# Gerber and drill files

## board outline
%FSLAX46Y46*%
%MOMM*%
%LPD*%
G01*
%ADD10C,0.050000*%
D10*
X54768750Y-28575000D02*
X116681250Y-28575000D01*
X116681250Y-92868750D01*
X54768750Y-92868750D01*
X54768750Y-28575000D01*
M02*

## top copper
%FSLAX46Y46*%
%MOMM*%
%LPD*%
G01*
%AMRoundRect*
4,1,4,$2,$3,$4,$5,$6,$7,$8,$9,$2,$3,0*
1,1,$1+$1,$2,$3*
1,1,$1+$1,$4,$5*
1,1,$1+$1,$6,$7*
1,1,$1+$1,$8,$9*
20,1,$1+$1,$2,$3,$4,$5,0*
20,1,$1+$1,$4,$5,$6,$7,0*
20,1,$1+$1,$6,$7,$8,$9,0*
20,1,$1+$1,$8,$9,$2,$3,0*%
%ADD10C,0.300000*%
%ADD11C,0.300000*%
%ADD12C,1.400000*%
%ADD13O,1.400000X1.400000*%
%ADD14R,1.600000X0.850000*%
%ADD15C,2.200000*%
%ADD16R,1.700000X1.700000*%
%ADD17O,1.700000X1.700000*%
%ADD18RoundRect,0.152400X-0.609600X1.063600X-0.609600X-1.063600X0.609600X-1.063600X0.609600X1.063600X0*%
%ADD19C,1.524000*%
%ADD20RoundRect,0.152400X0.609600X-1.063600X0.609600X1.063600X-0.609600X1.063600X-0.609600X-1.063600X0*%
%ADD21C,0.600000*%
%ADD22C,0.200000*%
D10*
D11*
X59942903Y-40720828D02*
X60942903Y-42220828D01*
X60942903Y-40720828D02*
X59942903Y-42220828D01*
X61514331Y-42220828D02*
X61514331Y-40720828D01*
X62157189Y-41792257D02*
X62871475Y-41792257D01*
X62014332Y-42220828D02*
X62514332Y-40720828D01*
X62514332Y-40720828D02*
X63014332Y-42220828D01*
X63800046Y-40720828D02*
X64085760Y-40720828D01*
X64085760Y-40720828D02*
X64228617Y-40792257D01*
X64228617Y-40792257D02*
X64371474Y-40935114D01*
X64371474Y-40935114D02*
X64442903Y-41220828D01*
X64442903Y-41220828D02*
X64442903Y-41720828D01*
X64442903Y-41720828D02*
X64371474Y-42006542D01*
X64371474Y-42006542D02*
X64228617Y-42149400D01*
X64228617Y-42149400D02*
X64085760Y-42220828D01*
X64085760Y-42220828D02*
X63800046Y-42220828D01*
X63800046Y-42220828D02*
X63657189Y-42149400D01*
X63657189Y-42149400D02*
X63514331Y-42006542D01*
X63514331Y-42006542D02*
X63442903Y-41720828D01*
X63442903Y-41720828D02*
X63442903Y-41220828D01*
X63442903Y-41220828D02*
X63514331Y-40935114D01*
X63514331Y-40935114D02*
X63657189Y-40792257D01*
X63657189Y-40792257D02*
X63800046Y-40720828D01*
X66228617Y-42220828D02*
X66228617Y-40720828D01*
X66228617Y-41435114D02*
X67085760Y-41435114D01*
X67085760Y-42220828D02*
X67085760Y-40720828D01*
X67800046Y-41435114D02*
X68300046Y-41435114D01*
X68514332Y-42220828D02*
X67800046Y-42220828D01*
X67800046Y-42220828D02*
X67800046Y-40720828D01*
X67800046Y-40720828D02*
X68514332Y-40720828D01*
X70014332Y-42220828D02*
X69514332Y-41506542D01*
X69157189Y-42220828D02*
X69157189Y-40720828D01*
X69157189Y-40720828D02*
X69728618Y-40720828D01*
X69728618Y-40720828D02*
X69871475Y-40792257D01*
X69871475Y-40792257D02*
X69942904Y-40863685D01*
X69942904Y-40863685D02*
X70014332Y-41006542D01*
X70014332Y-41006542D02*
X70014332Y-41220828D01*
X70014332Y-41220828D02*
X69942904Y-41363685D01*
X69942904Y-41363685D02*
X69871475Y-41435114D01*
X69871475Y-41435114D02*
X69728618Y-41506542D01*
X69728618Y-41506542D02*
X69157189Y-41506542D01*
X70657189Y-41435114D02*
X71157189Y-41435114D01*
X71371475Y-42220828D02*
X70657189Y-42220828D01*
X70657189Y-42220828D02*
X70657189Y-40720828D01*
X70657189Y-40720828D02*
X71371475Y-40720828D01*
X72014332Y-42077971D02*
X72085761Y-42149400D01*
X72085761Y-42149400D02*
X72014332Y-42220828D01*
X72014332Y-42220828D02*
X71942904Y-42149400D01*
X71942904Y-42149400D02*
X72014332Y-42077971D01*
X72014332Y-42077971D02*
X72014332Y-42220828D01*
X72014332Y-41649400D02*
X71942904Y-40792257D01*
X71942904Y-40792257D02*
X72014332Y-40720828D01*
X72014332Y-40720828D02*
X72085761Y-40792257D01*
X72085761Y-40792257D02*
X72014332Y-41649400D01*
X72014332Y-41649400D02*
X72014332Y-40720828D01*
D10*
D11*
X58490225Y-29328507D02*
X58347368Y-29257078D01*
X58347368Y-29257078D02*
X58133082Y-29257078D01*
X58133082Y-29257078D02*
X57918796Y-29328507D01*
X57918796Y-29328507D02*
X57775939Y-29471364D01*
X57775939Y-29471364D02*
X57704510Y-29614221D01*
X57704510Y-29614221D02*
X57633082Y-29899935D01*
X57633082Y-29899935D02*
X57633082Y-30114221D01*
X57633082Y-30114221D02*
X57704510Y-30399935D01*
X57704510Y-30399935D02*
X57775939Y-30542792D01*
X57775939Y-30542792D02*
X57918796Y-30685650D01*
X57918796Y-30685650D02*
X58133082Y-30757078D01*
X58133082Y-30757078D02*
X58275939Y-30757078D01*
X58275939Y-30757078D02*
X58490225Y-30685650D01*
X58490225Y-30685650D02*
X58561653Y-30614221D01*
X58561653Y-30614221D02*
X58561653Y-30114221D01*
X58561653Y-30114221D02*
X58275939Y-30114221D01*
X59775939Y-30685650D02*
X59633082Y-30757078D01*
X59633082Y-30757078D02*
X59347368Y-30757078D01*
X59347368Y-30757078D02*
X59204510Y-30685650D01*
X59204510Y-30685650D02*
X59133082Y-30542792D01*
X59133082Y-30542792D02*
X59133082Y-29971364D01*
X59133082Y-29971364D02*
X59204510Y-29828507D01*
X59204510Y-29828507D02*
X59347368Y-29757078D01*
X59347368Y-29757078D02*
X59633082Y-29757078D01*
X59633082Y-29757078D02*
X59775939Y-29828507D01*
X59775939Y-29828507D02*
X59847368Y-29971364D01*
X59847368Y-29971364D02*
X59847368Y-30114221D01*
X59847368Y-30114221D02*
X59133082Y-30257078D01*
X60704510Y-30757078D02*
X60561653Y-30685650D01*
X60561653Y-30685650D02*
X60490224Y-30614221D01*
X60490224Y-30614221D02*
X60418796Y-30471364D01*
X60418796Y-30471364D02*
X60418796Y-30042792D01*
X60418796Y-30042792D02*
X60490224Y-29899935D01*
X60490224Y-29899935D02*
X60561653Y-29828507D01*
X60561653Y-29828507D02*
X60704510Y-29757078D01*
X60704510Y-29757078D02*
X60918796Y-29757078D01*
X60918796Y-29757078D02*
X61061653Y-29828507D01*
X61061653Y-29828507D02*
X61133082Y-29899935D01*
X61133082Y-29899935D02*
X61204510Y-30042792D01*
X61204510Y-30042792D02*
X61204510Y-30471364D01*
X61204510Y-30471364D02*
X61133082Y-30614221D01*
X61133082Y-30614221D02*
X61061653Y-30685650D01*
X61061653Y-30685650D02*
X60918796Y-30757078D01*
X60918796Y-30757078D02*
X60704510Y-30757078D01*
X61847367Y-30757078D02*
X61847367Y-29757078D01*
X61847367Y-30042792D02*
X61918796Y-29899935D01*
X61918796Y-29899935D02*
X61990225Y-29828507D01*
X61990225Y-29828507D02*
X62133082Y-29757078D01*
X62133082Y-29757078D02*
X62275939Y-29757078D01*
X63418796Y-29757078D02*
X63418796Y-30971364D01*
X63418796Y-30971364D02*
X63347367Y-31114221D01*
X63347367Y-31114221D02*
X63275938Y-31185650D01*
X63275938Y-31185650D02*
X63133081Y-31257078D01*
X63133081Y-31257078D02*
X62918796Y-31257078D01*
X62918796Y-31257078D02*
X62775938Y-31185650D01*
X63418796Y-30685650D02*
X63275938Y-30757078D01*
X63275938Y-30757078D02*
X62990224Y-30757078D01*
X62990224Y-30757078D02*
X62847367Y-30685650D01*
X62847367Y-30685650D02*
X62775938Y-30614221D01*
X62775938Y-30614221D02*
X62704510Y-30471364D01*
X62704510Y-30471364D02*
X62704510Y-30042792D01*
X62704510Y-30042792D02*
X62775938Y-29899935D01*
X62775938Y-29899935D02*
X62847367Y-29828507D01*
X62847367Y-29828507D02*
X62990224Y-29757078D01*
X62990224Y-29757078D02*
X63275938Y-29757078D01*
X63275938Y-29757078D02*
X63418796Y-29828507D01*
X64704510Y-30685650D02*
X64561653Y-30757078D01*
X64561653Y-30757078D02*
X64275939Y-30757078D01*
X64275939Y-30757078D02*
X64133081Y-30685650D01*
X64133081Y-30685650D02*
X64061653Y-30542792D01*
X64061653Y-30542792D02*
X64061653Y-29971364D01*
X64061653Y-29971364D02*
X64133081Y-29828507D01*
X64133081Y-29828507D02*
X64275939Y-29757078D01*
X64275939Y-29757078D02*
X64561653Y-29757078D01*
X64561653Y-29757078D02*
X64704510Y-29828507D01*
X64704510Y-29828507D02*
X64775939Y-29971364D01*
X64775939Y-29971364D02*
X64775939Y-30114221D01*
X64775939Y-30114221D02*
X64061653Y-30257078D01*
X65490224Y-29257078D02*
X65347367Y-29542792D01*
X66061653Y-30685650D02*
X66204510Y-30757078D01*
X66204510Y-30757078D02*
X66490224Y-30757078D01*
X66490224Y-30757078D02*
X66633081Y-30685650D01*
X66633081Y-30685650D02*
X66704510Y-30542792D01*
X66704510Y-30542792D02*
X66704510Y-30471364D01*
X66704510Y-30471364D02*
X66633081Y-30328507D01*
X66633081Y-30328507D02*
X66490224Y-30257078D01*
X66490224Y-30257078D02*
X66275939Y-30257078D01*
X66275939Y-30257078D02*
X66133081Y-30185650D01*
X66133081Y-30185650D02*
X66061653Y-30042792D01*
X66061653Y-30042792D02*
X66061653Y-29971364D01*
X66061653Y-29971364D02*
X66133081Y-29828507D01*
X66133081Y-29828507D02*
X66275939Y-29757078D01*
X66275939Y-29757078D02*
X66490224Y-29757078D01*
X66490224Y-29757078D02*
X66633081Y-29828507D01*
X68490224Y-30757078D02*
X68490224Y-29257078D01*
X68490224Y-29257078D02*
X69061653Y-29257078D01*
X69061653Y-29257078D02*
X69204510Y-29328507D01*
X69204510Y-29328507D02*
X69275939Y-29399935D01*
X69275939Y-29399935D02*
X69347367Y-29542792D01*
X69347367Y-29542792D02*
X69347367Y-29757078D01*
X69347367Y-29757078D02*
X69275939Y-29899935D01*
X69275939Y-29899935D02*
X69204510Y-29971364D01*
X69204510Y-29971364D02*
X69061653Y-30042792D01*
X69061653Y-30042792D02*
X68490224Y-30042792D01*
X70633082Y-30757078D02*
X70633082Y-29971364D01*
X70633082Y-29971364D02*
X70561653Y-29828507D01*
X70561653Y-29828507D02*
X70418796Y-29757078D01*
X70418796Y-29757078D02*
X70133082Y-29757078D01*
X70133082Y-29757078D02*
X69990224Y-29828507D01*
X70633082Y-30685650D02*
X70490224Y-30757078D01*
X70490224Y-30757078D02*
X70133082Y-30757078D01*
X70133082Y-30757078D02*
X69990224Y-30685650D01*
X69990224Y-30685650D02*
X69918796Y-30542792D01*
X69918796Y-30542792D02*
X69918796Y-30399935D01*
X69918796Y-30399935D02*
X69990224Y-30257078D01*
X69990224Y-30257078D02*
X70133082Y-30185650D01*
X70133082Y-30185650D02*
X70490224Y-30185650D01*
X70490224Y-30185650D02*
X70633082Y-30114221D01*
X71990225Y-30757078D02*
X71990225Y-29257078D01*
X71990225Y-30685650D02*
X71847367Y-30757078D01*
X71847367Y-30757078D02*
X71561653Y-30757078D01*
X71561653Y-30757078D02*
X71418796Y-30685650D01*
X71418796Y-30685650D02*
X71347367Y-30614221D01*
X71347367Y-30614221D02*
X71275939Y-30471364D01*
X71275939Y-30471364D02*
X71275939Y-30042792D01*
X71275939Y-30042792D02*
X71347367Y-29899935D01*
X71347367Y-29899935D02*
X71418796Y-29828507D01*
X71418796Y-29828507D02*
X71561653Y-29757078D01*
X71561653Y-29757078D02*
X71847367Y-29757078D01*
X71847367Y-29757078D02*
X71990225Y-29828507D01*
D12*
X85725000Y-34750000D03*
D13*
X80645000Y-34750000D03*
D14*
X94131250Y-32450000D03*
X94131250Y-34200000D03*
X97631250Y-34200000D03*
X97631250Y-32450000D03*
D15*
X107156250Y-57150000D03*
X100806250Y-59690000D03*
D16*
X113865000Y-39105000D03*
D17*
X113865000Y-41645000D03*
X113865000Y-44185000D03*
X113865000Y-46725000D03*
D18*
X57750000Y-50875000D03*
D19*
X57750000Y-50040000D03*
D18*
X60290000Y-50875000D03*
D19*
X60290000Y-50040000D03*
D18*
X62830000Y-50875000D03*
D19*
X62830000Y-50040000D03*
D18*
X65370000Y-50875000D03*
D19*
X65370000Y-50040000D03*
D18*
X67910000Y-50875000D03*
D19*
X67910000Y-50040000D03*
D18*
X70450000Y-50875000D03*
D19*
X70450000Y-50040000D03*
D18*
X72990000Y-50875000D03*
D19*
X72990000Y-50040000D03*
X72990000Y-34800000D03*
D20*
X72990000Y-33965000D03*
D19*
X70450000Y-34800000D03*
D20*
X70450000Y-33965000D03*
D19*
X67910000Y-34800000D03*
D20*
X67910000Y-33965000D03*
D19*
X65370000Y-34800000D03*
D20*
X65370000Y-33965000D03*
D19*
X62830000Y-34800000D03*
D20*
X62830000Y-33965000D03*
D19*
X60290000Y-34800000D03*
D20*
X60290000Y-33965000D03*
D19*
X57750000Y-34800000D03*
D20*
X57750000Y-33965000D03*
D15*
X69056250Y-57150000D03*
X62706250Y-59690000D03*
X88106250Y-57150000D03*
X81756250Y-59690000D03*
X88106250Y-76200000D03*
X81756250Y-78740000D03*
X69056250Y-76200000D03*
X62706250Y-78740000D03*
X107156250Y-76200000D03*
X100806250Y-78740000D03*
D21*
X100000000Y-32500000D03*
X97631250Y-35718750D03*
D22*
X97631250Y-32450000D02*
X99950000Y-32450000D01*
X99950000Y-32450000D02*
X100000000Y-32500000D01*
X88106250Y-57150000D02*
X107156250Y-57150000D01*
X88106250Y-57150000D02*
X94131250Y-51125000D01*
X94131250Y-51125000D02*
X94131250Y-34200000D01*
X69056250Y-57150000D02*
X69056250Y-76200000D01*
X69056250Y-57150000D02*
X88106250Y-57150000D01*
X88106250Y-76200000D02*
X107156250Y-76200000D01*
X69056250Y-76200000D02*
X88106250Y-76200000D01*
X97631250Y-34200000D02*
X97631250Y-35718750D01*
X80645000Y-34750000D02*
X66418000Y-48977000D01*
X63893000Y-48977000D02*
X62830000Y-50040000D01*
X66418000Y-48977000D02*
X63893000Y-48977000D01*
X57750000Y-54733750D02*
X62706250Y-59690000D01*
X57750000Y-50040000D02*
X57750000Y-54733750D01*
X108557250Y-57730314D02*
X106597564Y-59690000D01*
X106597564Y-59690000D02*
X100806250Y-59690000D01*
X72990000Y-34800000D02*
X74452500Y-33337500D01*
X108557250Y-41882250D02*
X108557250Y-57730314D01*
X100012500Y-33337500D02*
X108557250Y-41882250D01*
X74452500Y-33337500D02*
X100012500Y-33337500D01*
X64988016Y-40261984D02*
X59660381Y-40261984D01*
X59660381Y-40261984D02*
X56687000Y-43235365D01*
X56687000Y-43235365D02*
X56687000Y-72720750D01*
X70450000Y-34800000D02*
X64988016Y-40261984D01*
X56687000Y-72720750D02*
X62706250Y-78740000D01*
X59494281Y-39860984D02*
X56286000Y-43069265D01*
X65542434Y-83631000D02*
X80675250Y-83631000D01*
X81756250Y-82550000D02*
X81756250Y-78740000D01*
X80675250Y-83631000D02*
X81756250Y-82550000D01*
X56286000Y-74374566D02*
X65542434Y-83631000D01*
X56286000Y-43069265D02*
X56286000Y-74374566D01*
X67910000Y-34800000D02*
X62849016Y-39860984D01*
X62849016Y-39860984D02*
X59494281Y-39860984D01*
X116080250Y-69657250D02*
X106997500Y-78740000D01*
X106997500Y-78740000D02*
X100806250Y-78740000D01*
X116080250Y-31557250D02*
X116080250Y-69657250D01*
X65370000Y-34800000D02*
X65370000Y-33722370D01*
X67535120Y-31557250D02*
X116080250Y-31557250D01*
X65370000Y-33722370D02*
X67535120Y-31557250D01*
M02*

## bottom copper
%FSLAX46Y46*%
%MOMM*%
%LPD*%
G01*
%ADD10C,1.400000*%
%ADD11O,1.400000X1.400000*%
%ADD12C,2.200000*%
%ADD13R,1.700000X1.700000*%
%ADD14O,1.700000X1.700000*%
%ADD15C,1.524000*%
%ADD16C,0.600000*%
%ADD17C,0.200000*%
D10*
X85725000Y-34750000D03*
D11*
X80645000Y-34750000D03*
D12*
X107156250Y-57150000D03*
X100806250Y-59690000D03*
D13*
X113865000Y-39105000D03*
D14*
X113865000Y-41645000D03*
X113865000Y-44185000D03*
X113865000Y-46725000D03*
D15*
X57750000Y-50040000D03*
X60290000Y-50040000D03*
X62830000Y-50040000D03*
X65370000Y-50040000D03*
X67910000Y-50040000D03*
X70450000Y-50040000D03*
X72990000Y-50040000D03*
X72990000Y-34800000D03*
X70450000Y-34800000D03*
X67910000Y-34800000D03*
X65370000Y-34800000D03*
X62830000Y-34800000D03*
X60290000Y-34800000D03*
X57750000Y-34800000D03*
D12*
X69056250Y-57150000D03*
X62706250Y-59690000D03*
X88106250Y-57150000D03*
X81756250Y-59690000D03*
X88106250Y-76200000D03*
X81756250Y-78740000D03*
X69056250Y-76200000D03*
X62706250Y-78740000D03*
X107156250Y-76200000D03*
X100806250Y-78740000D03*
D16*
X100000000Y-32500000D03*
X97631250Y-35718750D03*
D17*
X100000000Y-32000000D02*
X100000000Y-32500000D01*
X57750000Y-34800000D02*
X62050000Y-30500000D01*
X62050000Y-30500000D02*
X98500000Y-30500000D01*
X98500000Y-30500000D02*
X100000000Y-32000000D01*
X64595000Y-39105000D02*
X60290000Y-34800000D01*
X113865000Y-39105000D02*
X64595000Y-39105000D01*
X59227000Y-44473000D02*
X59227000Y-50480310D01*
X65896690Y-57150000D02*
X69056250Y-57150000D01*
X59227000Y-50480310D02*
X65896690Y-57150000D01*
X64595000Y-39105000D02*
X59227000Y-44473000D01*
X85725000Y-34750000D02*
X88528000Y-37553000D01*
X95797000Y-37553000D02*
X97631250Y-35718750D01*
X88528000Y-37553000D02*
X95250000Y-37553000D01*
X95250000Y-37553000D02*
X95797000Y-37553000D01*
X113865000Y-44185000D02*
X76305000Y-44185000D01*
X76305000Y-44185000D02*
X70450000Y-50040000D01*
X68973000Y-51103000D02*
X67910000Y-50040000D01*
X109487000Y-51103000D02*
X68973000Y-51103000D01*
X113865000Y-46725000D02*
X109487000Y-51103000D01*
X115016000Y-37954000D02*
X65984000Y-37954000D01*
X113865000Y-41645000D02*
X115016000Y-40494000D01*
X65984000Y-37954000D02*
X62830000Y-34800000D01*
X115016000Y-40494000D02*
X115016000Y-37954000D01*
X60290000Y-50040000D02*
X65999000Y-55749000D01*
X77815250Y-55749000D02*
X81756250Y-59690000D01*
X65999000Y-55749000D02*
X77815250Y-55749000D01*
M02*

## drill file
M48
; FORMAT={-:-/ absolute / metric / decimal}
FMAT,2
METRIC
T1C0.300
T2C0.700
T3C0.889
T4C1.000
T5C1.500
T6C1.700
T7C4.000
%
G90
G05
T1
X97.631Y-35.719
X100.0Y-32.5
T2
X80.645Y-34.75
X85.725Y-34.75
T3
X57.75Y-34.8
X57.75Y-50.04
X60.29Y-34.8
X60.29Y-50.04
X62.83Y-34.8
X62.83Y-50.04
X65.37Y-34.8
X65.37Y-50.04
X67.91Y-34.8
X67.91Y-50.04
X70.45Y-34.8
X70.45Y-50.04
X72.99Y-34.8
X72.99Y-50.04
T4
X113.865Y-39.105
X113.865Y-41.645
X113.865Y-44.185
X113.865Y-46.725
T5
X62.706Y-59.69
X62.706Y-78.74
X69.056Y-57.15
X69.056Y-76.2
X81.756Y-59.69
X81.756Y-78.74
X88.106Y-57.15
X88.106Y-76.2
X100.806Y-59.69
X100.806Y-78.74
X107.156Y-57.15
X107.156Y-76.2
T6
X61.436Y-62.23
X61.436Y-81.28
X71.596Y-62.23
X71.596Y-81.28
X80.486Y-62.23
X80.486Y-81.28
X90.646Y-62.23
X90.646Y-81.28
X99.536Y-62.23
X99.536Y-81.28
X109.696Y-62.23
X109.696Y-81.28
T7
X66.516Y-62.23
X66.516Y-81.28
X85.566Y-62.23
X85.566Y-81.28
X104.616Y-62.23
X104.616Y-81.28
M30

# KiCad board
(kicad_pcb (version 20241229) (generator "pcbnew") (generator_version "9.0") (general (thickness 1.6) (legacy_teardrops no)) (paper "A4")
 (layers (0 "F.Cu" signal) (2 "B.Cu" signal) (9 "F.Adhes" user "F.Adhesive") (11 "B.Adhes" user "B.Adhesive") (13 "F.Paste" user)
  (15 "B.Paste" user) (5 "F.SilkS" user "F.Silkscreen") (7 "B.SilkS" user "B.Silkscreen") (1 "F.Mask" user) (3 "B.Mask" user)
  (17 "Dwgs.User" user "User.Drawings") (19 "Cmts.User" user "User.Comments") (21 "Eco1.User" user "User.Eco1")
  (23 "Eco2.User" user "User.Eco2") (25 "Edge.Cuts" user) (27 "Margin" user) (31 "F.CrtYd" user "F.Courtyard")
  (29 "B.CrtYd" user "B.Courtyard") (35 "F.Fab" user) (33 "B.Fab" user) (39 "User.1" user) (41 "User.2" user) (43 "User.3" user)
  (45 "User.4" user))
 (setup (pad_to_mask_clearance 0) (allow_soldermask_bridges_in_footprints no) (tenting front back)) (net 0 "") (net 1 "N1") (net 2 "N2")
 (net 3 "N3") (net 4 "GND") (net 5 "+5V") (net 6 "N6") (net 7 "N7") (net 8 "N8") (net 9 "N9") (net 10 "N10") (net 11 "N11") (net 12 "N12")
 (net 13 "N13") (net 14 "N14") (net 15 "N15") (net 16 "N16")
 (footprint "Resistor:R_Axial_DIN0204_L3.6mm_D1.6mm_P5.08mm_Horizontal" (layer "F.Cu") (at 85.725 34.75 180)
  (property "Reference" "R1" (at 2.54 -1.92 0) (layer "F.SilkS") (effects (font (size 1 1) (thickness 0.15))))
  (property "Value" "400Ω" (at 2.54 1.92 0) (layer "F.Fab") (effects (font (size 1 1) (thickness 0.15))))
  (pad "1" thru_hole circle (at 0 0 180) (size 1.4 1.4) (drill 0.7) (layers "*.Cu" "*.Mask") (remove_unused_layers no) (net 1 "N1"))
  (pad "2" thru_hole oval (at 5.08 0 180) (size 1.4 1.4) (drill 0.7) (layers "*.Cu" "*.Mask") (remove_unused_layers no) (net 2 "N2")))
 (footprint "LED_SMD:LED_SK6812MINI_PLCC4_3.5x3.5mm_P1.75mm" (layer "F.Cu") (at 95.88125 33.325)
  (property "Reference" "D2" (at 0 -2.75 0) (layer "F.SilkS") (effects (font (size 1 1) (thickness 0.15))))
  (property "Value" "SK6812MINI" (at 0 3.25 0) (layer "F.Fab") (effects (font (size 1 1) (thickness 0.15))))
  (pad "1" smd rect (at -1.75 -0.875) (size 1.6 0.85) (layers "F.Cu" "F.Mask" "F.Paste") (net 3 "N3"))
  (pad "2" smd rect (at -1.75 0.875) (size 1.6 0.85) (layers "F.Cu" "F.Mask" "F.Paste") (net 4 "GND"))
  (pad "3" smd rect (at 1.75 0.875) (size 1.6 0.85) (layers "F.Cu" "F.Mask" "F.Paste") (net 1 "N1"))
  (pad "4" smd rect (at 1.75 -0.875) (size 1.6 0.85) (layers "F.Cu" "F.Mask" "F.Paste") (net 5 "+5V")))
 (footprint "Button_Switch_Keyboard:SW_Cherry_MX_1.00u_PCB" (layer "F.Cu") (at 107.15625 57.15)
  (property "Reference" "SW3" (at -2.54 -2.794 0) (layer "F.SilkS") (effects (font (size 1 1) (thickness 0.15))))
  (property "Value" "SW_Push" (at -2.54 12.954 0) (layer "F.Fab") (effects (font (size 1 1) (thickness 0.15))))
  (pad "" np_thru_hole circle (at -7.62 5.08) (size 1.7 1.7) (drill 1.7) (layers "*.Cu" "*.Mask"))
  (pad "" np_thru_hole circle (at -2.54 5.08) (size 4 4) (drill 4) (layers "*.Cu" "*.Mask"))
  (pad "" np_thru_hole circle (at 2.54 5.08) (size 1.7 1.7) (drill 1.7) (layers "*.Cu" "*.Mask"))
  (pad "1" thru_hole circle (at 0 0) (size 2.2 2.2) (drill 1.5) (layers "*.Cu" "*.Mask") (remove_unused_layers no) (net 4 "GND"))
  (pad "2" thru_hole circle (at -6.35 2.54) (size 2.2 2.2) (drill 1.5) (layers "*.Cu" "*.Mask") (remove_unused_layers no) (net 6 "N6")))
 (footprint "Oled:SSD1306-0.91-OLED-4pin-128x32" (layer "F.Cu") (at 77.365 36.915)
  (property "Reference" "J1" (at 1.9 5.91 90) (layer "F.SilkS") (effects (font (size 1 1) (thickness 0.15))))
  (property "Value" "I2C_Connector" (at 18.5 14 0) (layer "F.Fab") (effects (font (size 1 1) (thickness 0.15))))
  (pad "1" thru_hole rect (at 36.5 2.19) (size 1.7 1.7) (drill 1) (layers "*.Cu" "*.Mask") (remove_unused_layers no) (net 4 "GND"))
  (pad "2" thru_hole oval (at 36.5 4.73) (size 1.7 1.7) (drill 1) (layers "*.Cu" "*.Mask") (remove_unused_layers no) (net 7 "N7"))
  (pad "3" thru_hole oval (at 36.5 7.27) (size 1.7 1.7) (drill 1) (layers "*.Cu" "*.Mask") (remove_unused_layers no) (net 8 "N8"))
  (pad "4" thru_hole oval (at 36.5 9.81) (size 1.7 1.7) (drill 1) (layers "*.Cu" "*.Mask") (remove_unused_layers no) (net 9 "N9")))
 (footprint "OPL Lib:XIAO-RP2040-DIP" (layer "F.Cu") (at 65.37 42.42 90)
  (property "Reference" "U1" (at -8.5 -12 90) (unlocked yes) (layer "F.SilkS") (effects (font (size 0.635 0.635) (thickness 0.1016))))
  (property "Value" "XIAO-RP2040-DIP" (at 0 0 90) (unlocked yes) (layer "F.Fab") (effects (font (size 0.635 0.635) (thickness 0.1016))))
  (pad "1" smd roundrect (at -8.455 -7.62 270) (size 2.432 1.524) (layers "F.Cu" "F.Mask") (roundrect_rratio 0.1) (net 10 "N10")
   (thermal_bridge_angle 45))
  (pad "1" thru_hole circle (at -7.62 -7.62 270) (size 1.524 1.524) (drill 0.889) (layers "*.Cu" "*.Mask") (remove_unused_layers no)
   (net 10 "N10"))
  (pad "2" smd roundrect (at -8.455 -5.08 270) (size 2.432 1.524) (layers "F.Cu" "F.Mask") (roundrect_rratio 0.1) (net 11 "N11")
   (thermal_bridge_angle 45))
  (pad "2" thru_hole circle (at -7.62 -5.08 270) (size 1.524 1.524) (drill 0.889) (layers "*.Cu" "*.Mask") (remove_unused_layers no)
   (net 11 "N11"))
  (pad "3" smd roundrect (at -8.455 -2.54 270) (size 2.432 1.524) (layers "F.Cu" "F.Mask") (roundrect_rratio 0.1) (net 2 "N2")
   (thermal_bridge_angle 45))
  (pad "3" thru_hole circle (at -7.62 -2.54 270) (size 1.524 1.524) (drill 0.889) (layers "*.Cu" "*.Mask") (remove_unused_layers no)
   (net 2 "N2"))
  (pad "4" smd roundrect (at -8.455 0 270) (size 2.432 1.524) (layers "F.Cu" "F.Mask") (roundrect_rratio 0.1) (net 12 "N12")
   (thermal_bridge_angle 45))
  (pad "4" thru_hole circle (at -7.62 0 270) (size 1.524 1.524) (drill 0.889) (layers "*.Cu" "*.Mask") (remove_unused_layers no)
   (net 12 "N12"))
  (pad "5" smd roundrect (at -8.455 2.54 270) (size 2.432 1.524) (layers "F.Cu" "F.Mask") (roundrect_rratio 0.1) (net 9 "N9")
   (thermal_bridge_angle 45))
  (pad "5" thru_hole circle (at -7.62 2.54 270) (size 1.524 1.524) (drill 0.889) (layers "*.Cu" "*.Mask") (remove_unused_layers no)
   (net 9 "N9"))
  (pad "6" smd roundrect (at -8.455 5.08 270) (size 2.432 1.524) (layers "F.Cu" "F.Mask") (roundrect_rratio 0.1) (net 8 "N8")
   (thermal_bridge_angle 45))
  (pad "6" thru_hole circle (at -7.62 5.08 270) (size 1.524 1.524) (drill 0.889) (layers "*.Cu" "*.Mask") (remove_unused_layers no)
   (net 8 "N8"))
  (pad "7" smd roundrect (at -8.455 7.62 270) (size 2.432 1.524) (layers "F.Cu" "F.Mask") (roundrect_rratio 0.1) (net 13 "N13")
   (thermal_bridge_angle 45))
  (pad "7" thru_hole circle (at -7.62 7.62 270) (size 1.524 1.524) (drill 0.889) (layers "*.Cu" "*.Mask") (remove_unused_layers no)
   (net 13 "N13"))
  (pad "8" thru_hole circle (at 7.62 7.62 90) (size 1.524 1.524) (drill 0.889) (layers "*.Cu" "*.Mask") (remove_unused_layers no)
   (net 6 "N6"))
  (pad "8" smd roundrect (at 8.455 7.62 90) (size 2.432 1.524) (layers "F.Cu" "F.Mask") (roundrect_rratio 0.1) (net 6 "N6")
   (thermal_bridge_angle 45))
  (pad "9" thru_hole circle (at 7.62 5.08 90) (size 1.524 1.524) (drill 0.889) (layers "*.Cu" "*.Mask") (remove_unused_layers no)
   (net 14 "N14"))
  (pad "9" smd roundrect (at 8.455 5.08 90) (size 2.432 1.524) (layers "F.Cu" "F.Mask") (roundrect_rratio 0.1) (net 14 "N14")
   (thermal_bridge_angle 45))
  (pad "10" thru_hole circle (at 7.62 2.54 90) (size 1.524 1.524) (drill 0.889) (layers "*.Cu" "*.Mask") (remove_unused_layers no)
   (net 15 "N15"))
  (pad "10" smd roundrect (at 8.455 2.54 90) (size 2.432 1.524) (layers "F.Cu" "F.Mask") (roundrect_rratio 0.1) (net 15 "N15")
   (thermal_bridge_angle 45))
  (pad "11" thru_hole circle (at 7.62 0 90) (size 1.524 1.524) (drill 0.889) (layers "*.Cu" "*.Mask") (remove_unused_layers no)
   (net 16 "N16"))
  (pad "11" smd roundrect (at 8.455 0 90) (size 2.432 1.524) (layers "F.Cu" "F.Mask") (roundrect_rratio 0.1) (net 16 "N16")
   (thermal_bridge_angle 45))
  (pad "12" thru_hole circle (at 7.62 -2.54 90) (size 1.524 1.524) (drill 0.889) (layers "*.Cu" "*.Mask") (remove_unused_layers no)
   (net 7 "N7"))
  (pad "12" smd roundrect (at 8.455 -2.54 90) (size 2.432 1.524) (layers "F.Cu" "F.Mask") (roundrect_rratio 0.1) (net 7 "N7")
   (thermal_bridge_angle 45))
  (pad "13" thru_hole circle (at 7.62 -5.08 90) (size 1.524 1.524) (drill 0.889) (layers "*.Cu" "*.Mask") (remove_unused_layers no)
   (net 4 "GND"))
  (pad "13" smd roundrect (at 8.455 -5.08 90) (size 2.432 1.524) (layers "F.Cu" "F.Mask") (roundrect_rratio 0.1) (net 4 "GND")
   (thermal_bridge_angle 45))
  (pad "14" thru_hole circle (at 7.62 -7.62 90) (size 1.524 1.524) (drill 0.889) (layers "*.Cu" "*.Mask") (remove_unused_layers no)
   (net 5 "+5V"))
  (pad "14" smd roundrect (at 8.455 -7.62 90) (size 2.432 1.524) (layers "F.Cu" "F.Mask") (roundrect_rratio 0.1) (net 5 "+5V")
   (thermal_bridge_angle 45)))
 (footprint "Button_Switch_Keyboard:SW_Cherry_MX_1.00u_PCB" (layer "F.Cu") (at 69.05625 57.15)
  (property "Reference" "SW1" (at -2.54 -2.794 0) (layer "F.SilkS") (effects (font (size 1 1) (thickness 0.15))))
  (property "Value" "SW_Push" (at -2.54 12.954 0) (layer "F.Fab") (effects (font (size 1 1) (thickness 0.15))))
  (pad "" np_thru_hole circle (at -7.62 5.08) (size 1.7 1.7) (drill 1.7) (layers "*.Cu" "*.Mask"))
  (pad "" np_thru_hole circle (at -2.54 5.08) (size 4 4) (drill 4) (layers "*.Cu" "*.Mask"))
  (pad "" np_thru_hole circle (at 2.54 5.08) (size 1.7 1.7) (drill 1.7) (layers "*.Cu" "*.Mask"))
  (pad "1" thru_hole circle (at 0 0) (size 2.2 2.2) (drill 1.5) (layers "*.Cu" "*.Mask") (remove_unused_layers no) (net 4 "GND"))
  (pad "2" thru_hole circle (at -6.35 2.54) (size 2.2 2.2) (drill 1.5) (layers "*.Cu" "*.Mask") (remove_unused_layers no) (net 10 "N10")))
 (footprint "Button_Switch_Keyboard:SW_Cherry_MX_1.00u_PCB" (layer "F.Cu") (at 88.10625 57.15)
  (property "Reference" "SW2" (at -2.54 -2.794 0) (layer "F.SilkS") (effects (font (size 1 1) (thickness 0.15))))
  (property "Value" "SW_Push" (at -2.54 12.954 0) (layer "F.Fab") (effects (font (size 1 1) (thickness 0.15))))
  (pad "" np_thru_hole circle (at -7.62 5.08) (size 1.7 1.7) (drill 1.7) (layers "*.Cu" "*.Mask"))
  (pad "" np_thru_hole circle (at -2.54 5.08) (size 4 4) (drill 4) (layers "*.Cu" "*.Mask"))
  (pad "" np_thru_hole circle (at 2.54 5.08) (size 1.7 1.7) (drill 1.7) (layers "*.Cu" "*.Mask"))
  (pad "1" thru_hole circle (at 0 0) (size 2.2 2.2) (drill 1.5) (layers "*.Cu" "*.Mask") (remove_unused_layers no) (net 4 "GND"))
  (pad "2" thru_hole circle (at -6.35 2.54) (size 2.2 2.2) (drill 1.5) (layers "*.Cu" "*.Mask") (remove_unused_layers no) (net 11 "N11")))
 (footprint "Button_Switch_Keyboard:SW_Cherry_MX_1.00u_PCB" (layer "F.Cu") (at 88.10625 76.2)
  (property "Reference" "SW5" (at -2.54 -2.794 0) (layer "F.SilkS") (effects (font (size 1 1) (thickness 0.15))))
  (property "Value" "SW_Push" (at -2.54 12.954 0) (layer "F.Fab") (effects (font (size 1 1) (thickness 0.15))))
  (pad "" np_thru_hole circle (at -7.62 5.08) (size 1.7 1.7) (drill 1.7) (layers "*.Cu" "*.Mask"))
  (pad "" np_thru_hole circle (at -2.54 5.08) (size 4 4) (drill 4) (layers "*.Cu" "*.Mask"))
  (pad "" np_thru_hole circle (at 2.54 5.08) (size 1.7 1.7) (drill 1.7) (layers "*.Cu" "*.Mask"))
  (pad "1" thru_hole circle (at 0 0) (size 2.2 2.2) (drill 1.5) (layers "*.Cu" "*.Mask") (remove_unused_layers no) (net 4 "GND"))
  (pad "2" thru_hole circle (at -6.35 2.54) (size 2.2 2.2) (drill 1.5) (layers "*.Cu" "*.Mask") (remove_unused_layers no) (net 15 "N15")))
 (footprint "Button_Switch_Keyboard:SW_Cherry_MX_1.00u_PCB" (layer "F.Cu") (at 69.05625 76.2)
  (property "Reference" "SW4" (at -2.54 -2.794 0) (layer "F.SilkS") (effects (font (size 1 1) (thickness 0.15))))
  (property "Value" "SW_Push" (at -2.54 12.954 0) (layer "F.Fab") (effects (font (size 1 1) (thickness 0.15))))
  (pad "" np_thru_hole circle (at -7.62 5.08) (size 1.7 1.7) (drill 1.7) (layers "*.Cu" "*.Mask"))
  (pad "" np_thru_hole circle (at -2.54 5.08) (size 4 4) (drill 4) (layers "*.Cu" "*.Mask"))
  (pad "" np_thru_hole circle (at 2.54 5.08) (size 1.7 1.7) (drill 1.7) (layers "*.Cu" "*.Mask"))
  (pad "1" thru_hole circle (at 0 0) (size 2.2 2.2) (drill 1.5) (layers "*.Cu" "*.Mask") (remove_unused_layers no) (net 4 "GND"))
  (pad "2" thru_hole circle (at -6.35 2.54) (size 2.2 2.2) (drill 1.5) (layers "*.Cu" "*.Mask") (remove_unused_layers no) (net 14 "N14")))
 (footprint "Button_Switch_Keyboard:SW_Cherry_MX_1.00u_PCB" (layer "F.Cu") (at 107.15625 76.2)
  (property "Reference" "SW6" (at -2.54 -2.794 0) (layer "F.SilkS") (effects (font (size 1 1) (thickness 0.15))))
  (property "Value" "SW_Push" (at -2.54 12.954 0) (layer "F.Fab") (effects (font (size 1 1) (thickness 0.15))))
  (pad "" np_thru_hole circle (at -7.62 5.08) (size 1.7 1.7) (drill 1.7) (layers "*.Cu" "*.Mask"))
  (pad "" np_thru_hole circle (at -2.54 5.08) (size 4 4) (drill 4) (layers "*.Cu" "*.Mask"))
  (pad "" np_thru_hole circle (at 2.54 5.08) (size 1.7 1.7) (drill 1.7) (layers "*.Cu" "*.Mask"))
  (pad "1" thru_hole circle (at 0 0) (size 2.2 2.2) (drill 1.5) (layers "*.Cu" "*.Mask") (remove_unused_layers no) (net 4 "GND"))
  (pad "2" thru_hole circle (at -6.35 2.54) (size 2.2 2.2) (drill 1.5) (layers "*.Cu" "*.Mask") (remove_unused_layers no) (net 16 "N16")))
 (gr_rect (start 54.76875 28.575) (end 116.68125 92.86875) (stroke (width 0.05) (type default)) (fill no) (layer "Edge.Cuts"))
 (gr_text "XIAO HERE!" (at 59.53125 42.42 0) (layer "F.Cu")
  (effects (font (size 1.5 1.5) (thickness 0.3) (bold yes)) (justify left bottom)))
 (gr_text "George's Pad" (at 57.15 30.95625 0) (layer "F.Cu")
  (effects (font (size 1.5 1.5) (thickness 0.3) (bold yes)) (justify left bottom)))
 (segment (start 97.63125 32.45) (end 99.95 32.45) (width 0.2) (layer "F.Cu") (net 5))
 (segment (start 99.95 32.45) (end 100 32.5) (width 0.2) (layer "F.Cu") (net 5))
 (via (at 100 32.5) (size 0.6) (drill 0.3) (layers "F.Cu" "B.Cu") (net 5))
 (segment (start 100 32) (end 100 32.5) (width 0.2) (layer "B.Cu") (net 5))
 (segment (start 57.75 34.8) (end 62.05 30.5) (width 0.2) (layer "B.Cu") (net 5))
 (segment (start 62.05 30.5) (end 98.5 30.5) (width 0.2) (layer "B.Cu") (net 5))
 (segment (start 98.5 30.5) (end 100 32) (width 0.2) (layer "B.Cu") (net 5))
 (segment (start 88.10625 57.15) (end 107.15625 57.15) (width 0.2) (layer "F.Cu") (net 4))
 (segment (start 88.10625 57.15) (end 94.13125 51.125) (width 0.2) (layer "F.Cu") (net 4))
 (segment (start 94.13125 51.125) (end 94.13125 34.2) (width 0.2) (layer "F.Cu") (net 4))
 (segment (start 69.05625 57.15) (end 69.05625 76.2) (width 0.2) (layer "F.Cu") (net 4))
 (segment (start 69.05625 57.15) (end 88.10625 57.15) (width 0.2) (layer "F.Cu") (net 4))
 (segment (start 88.10625 76.2) (end 107.15625 76.2) (width 0.2) (layer "F.Cu") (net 4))
 (segment (start 69.05625 76.2) (end 88.10625 76.2) (width 0.2) (layer "F.Cu") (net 4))
 (segment (start 64.595 39.105) (end 60.29 34.8) (width 0.2) (layer "B.Cu") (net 4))
 (segment (start 113.865 39.105) (end 64.595 39.105) (width 0.2) (layer "B.Cu") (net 4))
 (segment (start 59.227 44.473) (end 59.227 50.48031) (width 0.2) (layer "B.Cu") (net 4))
 (segment (start 65.89669 57.15) (end 69.05625 57.15) (width 0.2) (layer "B.Cu") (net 4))
 (segment (start 59.227 50.48031) (end 65.89669 57.15) (width 0.2) (layer "B.Cu") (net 4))
 (segment (start 64.595 39.105) (end 59.227 44.473) (width 0.2) (layer "B.Cu") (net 4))
 (segment (start 97.63125 34.2) (end 97.63125 35.71875) (width 0.2) (layer "F.Cu") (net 1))
 (via (at 97.63125 35.71875) (size 0.6) (drill 0.3) (layers "F.Cu" "B.Cu") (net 1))
 (segment (start 85.725 34.75) (end 88.528 37.553) (width 0.2) (layer "B.Cu") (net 1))
 (segment (start 95.797 37.553) (end 97.63125 35.71875) (width 0.2) (layer "B.Cu") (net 1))
 (segment (start 88.528 37.553) (end 95.25 37.553) (width 0.2) (layer "B.Cu") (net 1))
 (segment (start 95.25 37.553) (end 95.797 37.553) (width 0.2) (layer "B.Cu") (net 1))
 (segment (start 113.865 44.185) (end 76.305 44.185) (width 0.2) (layer "B.Cu") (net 8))
 (segment (start 76.305 44.185) (end 70.45 50.04) (width 0.2) (layer "B.Cu") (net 8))
 (segment (start 68.973 51.103) (end 67.91 50.04) (width 0.2) (layer "B.Cu") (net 9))
 (segment (start 109.487 51.103) (end 68.973 51.103) (width 0.2) (layer "B.Cu") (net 9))
 (segment (start 113.865 46.725) (end 109.487 51.103) (width 0.2) (layer "B.Cu") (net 9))
 (segment (start 115.016 37.954) (end 65.984 37.954) (width 0.2) (layer "B.Cu") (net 7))
 (segment (start 113.865 41.645) (end 115.016 40.494) (width 0.2) (layer "B.Cu") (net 7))
 (segment (start 65.984 37.954) (end 62.83 34.8) (width 0.2) (layer "B.Cu") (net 7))
 (segment (start 115.016 40.494) (end 115.016 37.954) (width 0.2) (layer "B.Cu") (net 7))
 (segment (start 80.645 34.75) (end 66.418 48.977) (width 0.2) (layer "F.Cu") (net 2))
 (segment (start 63.893 48.977) (end 62.83 50.04) (width 0.2) (layer "F.Cu") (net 2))
 (segment (start 66.418 48.977) (end 63.893 48.977) (width 0.2) (layer "F.Cu") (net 2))
 (segment (start 57.75 54.73375) (end 62.70625 59.69) (width 0.2) (layer "F.Cu") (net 10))
 (segment (start 57.75 50.04) (end 57.75 54.73375) (width 0.2) (layer "F.Cu") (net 10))
 (segment (start 60.29 50.04) (end 65.999 55.749) (width 0.2) (layer "B.Cu") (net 11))
 (segment (start 77.81525 55.749) (end 81.75625 59.69) (width 0.2) (layer "B.Cu") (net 11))
 (segment (start 65.999 55.749) (end 77.81525 55.749) (width 0.2) (layer "B.Cu") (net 11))
 (segment (start 108.55725 57.730314) (end 106.597564 59.69) (width 0.2) (layer "F.Cu") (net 6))
 (segment (start 106.597564 59.69) (end 100.80625 59.69) (width 0.2) (layer "F.Cu") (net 6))
 (segment (start 72.99 34.8) (end 74.4525 33.3375) (width 0.2) (layer "F.Cu") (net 6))
 (segment (start 108.55725 41.88225) (end 108.55725 57.730314) (width 0.2) (layer "F.Cu") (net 6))
 (segment (start 100.0125 33.3375) (end 108.55725 41.88225) (width 0.2) (layer "F.Cu") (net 6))
 (segment (start 74.4525 33.3375) (end 100.0125 33.3375) (width 0.2) (layer "F.Cu") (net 6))
 (segment (start 64.988016 40.261984) (end 59.660381 40.261984) (width 0.2) (layer "F.Cu") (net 14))
 (segment (start 59.660381 40.261984) (end 56.687 43.235365) (width 0.2) (layer "F.Cu") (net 14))
 (segment (start 56.687 43.235365) (end 56.687 72.72075) (width 0.2) (layer "F.Cu") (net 14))
 (segment (start 70.45 34.8) (end 64.988016 40.261984) (width 0.2) (layer "F.Cu") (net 14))
 (segment (start 56.687 72.72075) (end 62.70625 78.74) (width 0.2) (layer "F.Cu") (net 14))
 (segment (start 59.494281 39.860984) (end 56.286 43.069265) (width 0.2) (layer "F.Cu") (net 15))
 (segment (start 65.542434 83.631) (end 80.67525 83.631) (width 0.2) (layer "F.Cu") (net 15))
 (segment (start 81.75625 82.55) (end 81.75625 78.74) (width 0.2) (layer "F.Cu") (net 15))
 (segment (start 80.67525 83.631) (end 81.75625 82.55) (width 0.2) (layer "F.Cu") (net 15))
 (segment (start 56.286 74.374566) (end 65.542434 83.631) (width 0.2) (layer "F.Cu") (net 15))
 (segment (start 56.286 43.069265) (end 56.286 74.374566) (width 0.2) (layer "F.Cu") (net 15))
 (segment (start 67.91 34.8) (end 62.849016 39.860984) (width 0.2) (layer "F.Cu") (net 15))
 (segment (start 62.849016 39.860984) (end 59.494281 39.860984) (width 0.2) (layer "F.Cu") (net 15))
 (segment (start 116.08025 69.65725) (end 106.9975 78.74) (width 0.2) (layer "F.Cu") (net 16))
 (segment (start 106.9975 78.74) (end 100.80625 78.74) (width 0.2) (layer "F.Cu") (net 16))
 (segment (start 116.08025 31.55725) (end 116.08025 69.65725) (width 0.2) (layer "F.Cu") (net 16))
 (segment (start 65.37 34.8) (end 65.37 33.72237) (width 0.2) (layer "F.Cu") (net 16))
 (segment (start 67.53512 31.55725) (end 116.08025 31.55725) (width 0.2) (layer "F.Cu") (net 16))
 (segment (start 65.37 33.72237) (end 67.53512 31.55725) (width 0.2) (layer "F.Cu") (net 16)))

